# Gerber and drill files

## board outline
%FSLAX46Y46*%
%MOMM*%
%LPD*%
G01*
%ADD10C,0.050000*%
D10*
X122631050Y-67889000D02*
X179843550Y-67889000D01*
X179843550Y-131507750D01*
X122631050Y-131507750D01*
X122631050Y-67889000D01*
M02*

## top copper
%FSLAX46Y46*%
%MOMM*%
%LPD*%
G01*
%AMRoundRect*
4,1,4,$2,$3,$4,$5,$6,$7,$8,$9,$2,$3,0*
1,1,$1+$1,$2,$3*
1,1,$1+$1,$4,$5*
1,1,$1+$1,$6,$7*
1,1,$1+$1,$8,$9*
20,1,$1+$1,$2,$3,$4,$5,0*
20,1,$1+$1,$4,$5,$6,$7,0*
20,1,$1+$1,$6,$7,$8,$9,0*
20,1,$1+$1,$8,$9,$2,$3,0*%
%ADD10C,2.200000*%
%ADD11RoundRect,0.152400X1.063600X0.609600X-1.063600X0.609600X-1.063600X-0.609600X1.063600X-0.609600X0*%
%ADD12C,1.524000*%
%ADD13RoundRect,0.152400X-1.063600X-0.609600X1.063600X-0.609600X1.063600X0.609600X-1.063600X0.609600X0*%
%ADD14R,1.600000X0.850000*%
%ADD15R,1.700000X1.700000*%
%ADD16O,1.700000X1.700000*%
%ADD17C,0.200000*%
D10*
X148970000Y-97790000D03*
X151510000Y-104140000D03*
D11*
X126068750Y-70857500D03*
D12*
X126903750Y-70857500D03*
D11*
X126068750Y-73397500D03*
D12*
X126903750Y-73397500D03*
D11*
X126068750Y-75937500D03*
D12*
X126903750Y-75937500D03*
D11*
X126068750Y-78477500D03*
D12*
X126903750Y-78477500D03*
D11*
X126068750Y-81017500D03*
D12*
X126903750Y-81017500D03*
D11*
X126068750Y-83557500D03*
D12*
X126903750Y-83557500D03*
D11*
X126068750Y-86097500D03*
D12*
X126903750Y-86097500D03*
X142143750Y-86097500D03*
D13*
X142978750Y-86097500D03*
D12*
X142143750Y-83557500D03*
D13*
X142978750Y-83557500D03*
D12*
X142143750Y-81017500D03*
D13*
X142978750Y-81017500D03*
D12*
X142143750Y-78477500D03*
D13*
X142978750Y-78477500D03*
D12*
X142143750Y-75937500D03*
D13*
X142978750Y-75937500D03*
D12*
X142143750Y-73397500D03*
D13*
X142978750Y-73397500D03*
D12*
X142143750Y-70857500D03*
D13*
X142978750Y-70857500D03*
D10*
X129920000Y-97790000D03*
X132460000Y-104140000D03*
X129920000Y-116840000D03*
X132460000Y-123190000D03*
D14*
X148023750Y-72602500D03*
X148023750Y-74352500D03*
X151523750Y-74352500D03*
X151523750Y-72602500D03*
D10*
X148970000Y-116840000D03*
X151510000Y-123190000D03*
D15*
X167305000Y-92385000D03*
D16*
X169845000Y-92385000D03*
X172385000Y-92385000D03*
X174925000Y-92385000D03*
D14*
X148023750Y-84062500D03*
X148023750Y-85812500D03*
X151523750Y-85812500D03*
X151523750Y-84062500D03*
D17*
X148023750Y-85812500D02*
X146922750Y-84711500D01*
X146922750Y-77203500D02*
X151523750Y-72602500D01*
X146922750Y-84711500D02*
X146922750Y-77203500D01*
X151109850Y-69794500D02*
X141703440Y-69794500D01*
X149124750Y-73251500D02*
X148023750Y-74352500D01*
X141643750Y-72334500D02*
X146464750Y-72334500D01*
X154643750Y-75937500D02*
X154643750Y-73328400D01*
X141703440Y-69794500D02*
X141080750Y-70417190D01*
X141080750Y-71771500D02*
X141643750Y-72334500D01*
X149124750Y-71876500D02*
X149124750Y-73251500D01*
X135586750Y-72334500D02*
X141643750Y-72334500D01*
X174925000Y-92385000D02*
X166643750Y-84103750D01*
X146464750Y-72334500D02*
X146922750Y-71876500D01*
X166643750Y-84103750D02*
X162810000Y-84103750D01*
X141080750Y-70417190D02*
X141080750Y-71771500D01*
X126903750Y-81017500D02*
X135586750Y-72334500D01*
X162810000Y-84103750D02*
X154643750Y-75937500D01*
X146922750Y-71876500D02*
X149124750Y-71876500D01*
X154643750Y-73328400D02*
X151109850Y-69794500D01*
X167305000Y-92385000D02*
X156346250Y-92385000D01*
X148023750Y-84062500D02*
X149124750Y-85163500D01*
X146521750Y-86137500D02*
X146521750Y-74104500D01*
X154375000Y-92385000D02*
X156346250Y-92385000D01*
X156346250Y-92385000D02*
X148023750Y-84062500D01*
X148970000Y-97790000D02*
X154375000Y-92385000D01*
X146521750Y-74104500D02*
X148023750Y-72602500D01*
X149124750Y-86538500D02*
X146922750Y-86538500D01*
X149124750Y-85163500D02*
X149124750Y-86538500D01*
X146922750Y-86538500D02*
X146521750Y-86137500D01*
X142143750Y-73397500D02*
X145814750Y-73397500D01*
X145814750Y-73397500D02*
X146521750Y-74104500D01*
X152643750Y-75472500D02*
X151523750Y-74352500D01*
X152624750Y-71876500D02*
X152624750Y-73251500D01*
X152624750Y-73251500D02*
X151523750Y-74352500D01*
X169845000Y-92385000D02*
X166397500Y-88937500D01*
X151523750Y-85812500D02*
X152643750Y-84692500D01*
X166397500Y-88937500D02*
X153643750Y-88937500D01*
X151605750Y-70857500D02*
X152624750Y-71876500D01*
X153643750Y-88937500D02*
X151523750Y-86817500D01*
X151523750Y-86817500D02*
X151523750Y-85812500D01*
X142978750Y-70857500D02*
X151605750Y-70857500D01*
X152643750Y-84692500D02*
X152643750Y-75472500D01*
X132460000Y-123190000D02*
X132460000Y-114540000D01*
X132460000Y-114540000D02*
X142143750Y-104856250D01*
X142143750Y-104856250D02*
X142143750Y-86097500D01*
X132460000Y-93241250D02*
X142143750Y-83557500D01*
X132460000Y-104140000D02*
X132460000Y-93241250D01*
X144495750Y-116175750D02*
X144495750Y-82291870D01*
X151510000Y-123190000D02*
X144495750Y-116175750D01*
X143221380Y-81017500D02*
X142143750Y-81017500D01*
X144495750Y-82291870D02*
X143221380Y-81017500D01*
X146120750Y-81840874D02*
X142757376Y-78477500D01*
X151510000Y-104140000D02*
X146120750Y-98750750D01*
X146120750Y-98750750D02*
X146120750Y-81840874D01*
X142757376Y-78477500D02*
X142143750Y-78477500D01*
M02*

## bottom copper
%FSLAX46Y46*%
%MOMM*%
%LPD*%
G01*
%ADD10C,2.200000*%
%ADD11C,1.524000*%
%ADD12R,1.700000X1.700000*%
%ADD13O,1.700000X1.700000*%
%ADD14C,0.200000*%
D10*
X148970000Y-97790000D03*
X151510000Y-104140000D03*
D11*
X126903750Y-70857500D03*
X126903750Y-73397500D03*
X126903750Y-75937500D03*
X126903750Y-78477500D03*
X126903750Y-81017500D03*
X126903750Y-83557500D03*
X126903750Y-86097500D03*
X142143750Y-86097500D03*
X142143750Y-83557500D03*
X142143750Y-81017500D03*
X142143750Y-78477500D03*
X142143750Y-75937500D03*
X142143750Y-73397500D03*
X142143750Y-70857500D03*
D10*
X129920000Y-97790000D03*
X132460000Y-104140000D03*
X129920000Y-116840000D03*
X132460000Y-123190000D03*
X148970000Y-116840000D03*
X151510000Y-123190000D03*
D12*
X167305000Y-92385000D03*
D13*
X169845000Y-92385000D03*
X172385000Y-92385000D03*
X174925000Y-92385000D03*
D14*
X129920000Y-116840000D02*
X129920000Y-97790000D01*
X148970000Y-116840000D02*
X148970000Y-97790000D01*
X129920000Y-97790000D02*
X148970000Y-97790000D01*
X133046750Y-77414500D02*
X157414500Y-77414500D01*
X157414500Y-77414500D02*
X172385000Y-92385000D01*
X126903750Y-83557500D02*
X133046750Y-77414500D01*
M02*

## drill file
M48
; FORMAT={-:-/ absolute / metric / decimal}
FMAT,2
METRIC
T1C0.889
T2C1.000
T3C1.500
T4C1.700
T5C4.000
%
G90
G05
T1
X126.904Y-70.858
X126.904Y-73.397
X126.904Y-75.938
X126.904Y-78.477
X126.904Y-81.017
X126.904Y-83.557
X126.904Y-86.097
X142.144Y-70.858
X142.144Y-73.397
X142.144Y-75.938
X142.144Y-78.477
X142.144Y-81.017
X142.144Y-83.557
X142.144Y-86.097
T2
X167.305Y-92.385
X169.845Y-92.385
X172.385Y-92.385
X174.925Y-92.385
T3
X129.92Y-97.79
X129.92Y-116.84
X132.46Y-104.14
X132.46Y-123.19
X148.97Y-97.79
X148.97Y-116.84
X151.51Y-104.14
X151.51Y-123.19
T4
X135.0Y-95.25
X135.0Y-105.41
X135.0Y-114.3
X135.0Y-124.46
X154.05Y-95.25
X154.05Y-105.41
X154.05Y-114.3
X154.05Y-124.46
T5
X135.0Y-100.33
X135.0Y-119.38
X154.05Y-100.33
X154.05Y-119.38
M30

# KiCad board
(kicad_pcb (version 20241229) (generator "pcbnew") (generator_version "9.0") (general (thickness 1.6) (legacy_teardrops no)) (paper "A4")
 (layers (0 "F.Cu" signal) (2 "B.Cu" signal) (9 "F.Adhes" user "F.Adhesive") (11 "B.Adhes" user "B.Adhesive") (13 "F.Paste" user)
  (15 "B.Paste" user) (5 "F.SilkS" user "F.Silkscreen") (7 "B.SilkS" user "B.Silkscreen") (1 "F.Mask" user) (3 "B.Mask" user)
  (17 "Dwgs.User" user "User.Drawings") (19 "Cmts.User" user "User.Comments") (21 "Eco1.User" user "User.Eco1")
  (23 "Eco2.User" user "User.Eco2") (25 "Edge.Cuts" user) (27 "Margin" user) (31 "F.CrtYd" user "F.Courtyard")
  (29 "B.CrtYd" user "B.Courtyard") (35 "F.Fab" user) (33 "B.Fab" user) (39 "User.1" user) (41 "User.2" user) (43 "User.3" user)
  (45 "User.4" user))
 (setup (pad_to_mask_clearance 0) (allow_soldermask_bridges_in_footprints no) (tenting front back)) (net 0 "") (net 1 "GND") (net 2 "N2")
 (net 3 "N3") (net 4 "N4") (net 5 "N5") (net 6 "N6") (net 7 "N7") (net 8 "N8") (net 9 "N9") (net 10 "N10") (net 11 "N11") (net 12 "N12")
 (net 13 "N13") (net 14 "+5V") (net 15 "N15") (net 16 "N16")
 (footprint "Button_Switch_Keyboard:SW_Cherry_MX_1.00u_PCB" (layer "F.Cu") (at 148.97 97.79 90)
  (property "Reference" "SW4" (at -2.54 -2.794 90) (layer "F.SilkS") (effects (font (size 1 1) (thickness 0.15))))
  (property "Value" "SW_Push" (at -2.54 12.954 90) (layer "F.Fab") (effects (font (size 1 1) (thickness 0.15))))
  (pad "" np_thru_hole circle (at -7.62 5.08 90) (size 1.7 1.7) (drill 1.7) (layers "*.Cu" "*.Mask"))
  (pad "" np_thru_hole circle (at -2.54 5.08 90) (size 4 4) (drill 4) (layers "*.Cu" "*.Mask"))
  (pad "" np_thru_hole circle (at 2.54 5.08 90) (size 1.7 1.7) (drill 1.7) (layers "*.Cu" "*.Mask"))
  (pad "1" thru_hole circle (at 0 0 90) (size 2.2 2.2) (drill 1.5) (layers "*.Cu" "*.Mask") (remove_unused_layers no) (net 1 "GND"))
  (pad "2" thru_hole circle (at -6.35 2.54 90) (size 2.2 2.2) (drill 1.5) (layers "*.Cu" "*.Mask") (remove_unused_layers no) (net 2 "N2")))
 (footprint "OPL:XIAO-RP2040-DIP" (layer "F.Cu") (at 134.52375 78.4775)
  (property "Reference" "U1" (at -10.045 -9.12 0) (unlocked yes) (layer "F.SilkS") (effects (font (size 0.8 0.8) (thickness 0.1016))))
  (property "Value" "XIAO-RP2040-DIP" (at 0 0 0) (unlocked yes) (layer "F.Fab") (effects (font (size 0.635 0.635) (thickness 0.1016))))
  (pad "1" smd roundrect (at -8.455 -7.62 180) (size 2.432 1.524) (layers "F.Cu" "F.Mask") (roundrect_rratio 0.1) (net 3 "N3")
   (thermal_bridge_angle 45))
  (pad "1" thru_hole circle (at -7.62 -7.62 180) (size 1.524 1.524) (drill 0.889) (layers "*.Cu" "*.Mask") (remove_unused_layers no)
   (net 3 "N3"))
  (pad "2" smd roundrect (at -8.455 -5.08 180) (size 2.432 1.524) (layers "F.Cu" "F.Mask") (roundrect_rratio 0.1) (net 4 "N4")
   (thermal_bridge_angle 45))
  (pad "2" thru_hole circle (at -7.62 -5.08 180) (size 1.524 1.524) (drill 0.889) (layers "*.Cu" "*.Mask") (remove_unused_layers no)
   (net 4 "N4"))
  (pad "3" smd roundrect (at -8.455 -2.54 180) (size 2.432 1.524) (layers "F.Cu" "F.Mask") (roundrect_rratio 0.1) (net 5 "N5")
   (thermal_bridge_angle 45))
  (pad "3" thru_hole circle (at -7.62 -2.54 180) (size 1.524 1.524) (drill 0.889) (layers "*.Cu" "*.Mask") (remove_unused_layers no)
   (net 5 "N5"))
  (pad "4" smd roundrect (at -8.455 0 180) (size 2.432 1.524) (layers "F.Cu" "F.Mask") (roundrect_rratio 0.1) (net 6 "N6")
   (thermal_bridge_angle 45))
  (pad "4" thru_hole circle (at -7.62 0 180) (size 1.524 1.524) (drill 0.889) (layers "*.Cu" "*.Mask") (remove_unused_layers no)
   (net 6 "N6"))
  (pad "5" smd roundrect (at -8.455 2.54 180) (size 2.432 1.524) (layers "F.Cu" "F.Mask") (roundrect_rratio 0.1) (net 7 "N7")
   (thermal_bridge_angle 45))
  (pad "5" thru_hole circle (at -7.62 2.54 180) (size 1.524 1.524) (drill 0.889) (layers "*.Cu" "*.Mask") (remove_unused_layers no)
   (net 7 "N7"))
  (pad "6" smd roundrect (at -8.455 5.08 180) (size 2.432 1.524) (layers "F.Cu" "F.Mask") (roundrect_rratio 0.1) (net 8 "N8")
   (thermal_bridge_angle 45))
  (pad "6" thru_hole circle (at -7.62 5.08 180) (size 1.524 1.524) (drill 0.889) (layers "*.Cu" "*.Mask") (remove_unused_layers no)
   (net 8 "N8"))
  (pad "7" smd roundrect (at -8.455 7.62 180) (size 2.432 1.524) (layers "F.Cu" "F.Mask") (roundrect_rratio 0.1) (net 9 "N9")
   (thermal_bridge_angle 45))
  (pad "7" thru_hole circle (at -7.62 7.62 180) (size 1.524 1.524) (drill 0.889) (layers "*.Cu" "*.Mask") (remove_unused_layers no)
   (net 9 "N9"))
  (pad "8" thru_hole circle (at 7.62 7.62) (size 1.524 1.524) (drill 0.889) (layers "*.Cu" "*.Mask") (remove_unused_layers no)
   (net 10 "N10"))
  (pad "8" smd roundrect (at 8.455 7.62) (size 2.432 1.524) (layers "F.Cu" "F.Mask") (roundrect_rratio 0.1) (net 10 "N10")
   (thermal_bridge_angle 45))
  (pad "9" thru_hole circle (at 7.62 5.08) (size 1.524 1.524) (drill 0.889) (layers "*.Cu" "*.Mask") (remove_unused_layers no)
   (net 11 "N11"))
  (pad "9" smd roundrect (at 8.455 5.08) (size 2.432 1.524) (layers "F.Cu" "F.Mask") (roundrect_rratio 0.1) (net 11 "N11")
   (thermal_bridge_angle 45))
  (pad "10" thru_hole circle (at 7.62 2.54) (size 1.524 1.524) (drill 0.889) (layers "*.Cu" "*.Mask") (remove_unused_layers no)
   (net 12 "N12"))
  (pad "10" smd roundrect (at 8.455 2.54) (size 2.432 1.524) (layers "F.Cu" "F.Mask") (roundrect_rratio 0.1) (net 12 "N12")
   (thermal_bridge_angle 45))
  (pad "11" thru_hole circle (at 7.62 0) (size 1.524 1.524) (drill 0.889) (layers "*.Cu" "*.Mask") (remove_unused_layers no) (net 2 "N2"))
  (pad "11" smd roundrect (at 8.455 0) (size 2.432 1.524) (layers "F.Cu" "F.Mask") (roundrect_rratio 0.1) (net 2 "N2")
   (thermal_bridge_angle 45))
  (pad "12" thru_hole circle (at 7.62 -2.54) (size 1.524 1.524) (drill 0.889) (layers "*.Cu" "*.Mask") (remove_unused_layers no)
   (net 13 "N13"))
  (pad "12" smd roundrect (at 8.455 -2.54) (size 2.432 1.524) (layers "F.Cu" "F.Mask") (roundrect_rratio 0.1) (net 13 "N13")
   (thermal_bridge_angle 45))
  (pad "13" thru_hole circle (at 7.62 -5.08) (size 1.524 1.524) (drill 0.889) (layers "*.Cu" "*.Mask") (remove_unused_layers no)
   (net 1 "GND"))
  (pad "13" smd roundrect (at 8.455 -5.08) (size 2.432 1.524) (layers "F.Cu" "F.Mask") (roundrect_rratio 0.1) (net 1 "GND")
   (thermal_bridge_angle 45))
  (pad "14" thru_hole circle (at 7.62 -7.62) (size 1.524 1.524) (drill 0.889) (layers "*.Cu" "*.Mask") (remove_unused_layers no)
   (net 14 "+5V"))
  (pad "14" smd roundrect (at 8.455 -7.62) (size 2.432 1.524) (layers "F.Cu" "F.Mask") (roundrect_rratio 0.1) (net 14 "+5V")
   (thermal_bridge_angle 45)))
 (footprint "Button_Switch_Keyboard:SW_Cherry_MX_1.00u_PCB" (layer "F.Cu") (at 129.92 97.79 90)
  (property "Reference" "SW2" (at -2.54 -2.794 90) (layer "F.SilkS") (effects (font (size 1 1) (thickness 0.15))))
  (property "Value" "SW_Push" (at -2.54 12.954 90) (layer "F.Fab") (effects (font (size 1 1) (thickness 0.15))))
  (pad "" np_thru_hole circle (at -7.62 5.08 90) (size 1.7 1.7) (drill 1.7) (layers "*.Cu" "*.Mask"))
  (pad "" np_thru_hole circle (at -2.54 5.08 90) (size 4 4) (drill 4) (layers "*.Cu" "*.Mask"))
  (pad "" np_thru_hole circle (at 2.54 5.08 90) (size 1.7 1.7) (drill 1.7) (layers "*.Cu" "*.Mask"))
  (pad "1" thru_hole circle (at 0 0 90) (size 2.2 2.2) (drill 1.5) (layers "*.Cu" "*.Mask") (remove_unused_layers no) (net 1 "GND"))
  (pad "2" thru_hole circle (at -6.35 2.54 90) (size 2.2 2.2) (drill 1.5) (layers "*.Cu" "*.Mask") (remove_unused_layers no) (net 11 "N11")))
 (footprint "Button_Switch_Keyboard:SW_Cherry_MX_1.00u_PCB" (layer "F.Cu") (at 129.92 116.84 90)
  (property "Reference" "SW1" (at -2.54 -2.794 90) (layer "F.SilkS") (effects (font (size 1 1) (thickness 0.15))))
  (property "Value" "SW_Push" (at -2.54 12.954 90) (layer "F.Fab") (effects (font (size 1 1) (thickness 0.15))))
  (pad "" np_thru_hole circle (at -7.62 5.08 90) (size 1.7 1.7) (drill 1.7) (layers "*.Cu" "*.Mask"))
  (pad "" np_thru_hole circle (at -2.54 5.08 90) (size 4 4) (drill 4) (layers "*.Cu" "*.Mask"))
  (pad "" np_thru_hole circle (at 2.54 5.08 90) (size 1.7 1.7) (drill 1.7) (layers "*.Cu" "*.Mask"))
  (pad "1" thru_hole circle (at 0 0 90) (size 2.2 2.2) (drill 1.5) (layers "*.Cu" "*.Mask") (remove_unused_layers no) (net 1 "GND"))
  (pad "2" thru_hole circle (at -6.35 2.54 90) (size 2.2 2.2) (drill 1.5) (layers "*.Cu" "*.Mask") (remove_unused_layers no) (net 10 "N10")))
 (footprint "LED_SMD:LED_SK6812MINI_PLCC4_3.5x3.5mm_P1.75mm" (layer "F.Cu") (at 149.77375 73.4775)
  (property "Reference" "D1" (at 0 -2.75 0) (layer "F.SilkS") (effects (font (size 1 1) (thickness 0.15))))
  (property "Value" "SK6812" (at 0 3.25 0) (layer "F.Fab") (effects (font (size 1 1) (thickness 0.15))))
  (pad "1" smd rect (at -1.75 -0.875) (size 1.6 0.85) (layers "F.Cu" "F.Mask" "F.Paste") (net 1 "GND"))
  (pad "2" smd rect (at -1.75 0.875) (size 1.6 0.85) (layers "F.Cu" "F.Mask" "F.Paste") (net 7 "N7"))
  (pad "3" smd rect (at 1.75 0.875) (size 1.6 0.85) (layers "F.Cu" "F.Mask" "F.Paste") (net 14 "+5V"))
  (pad "4" smd rect (at 1.75 -0.875) (size 1.6 0.85) (layers "F.Cu" "F.Mask" "F.Paste") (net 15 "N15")))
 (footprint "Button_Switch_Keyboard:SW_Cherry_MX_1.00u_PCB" (layer "F.Cu") (at 148.97 116.84 90)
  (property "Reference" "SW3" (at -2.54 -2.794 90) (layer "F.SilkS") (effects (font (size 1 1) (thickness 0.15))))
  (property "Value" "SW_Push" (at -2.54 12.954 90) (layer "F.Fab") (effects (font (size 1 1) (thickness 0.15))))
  (pad "" np_thru_hole circle (at -7.62 5.08 90) (size 1.7 1.7) (drill 1.7) (layers "*.Cu" "*.Mask"))
  (pad "" np_thru_hole circle (at -2.54 5.08 90) (size 4 4) (drill 4) (layers "*.Cu" "*.Mask"))
  (pad "" np_thru_hole circle (at 2.54 5.08 90) (size 1.7 1.7) (drill 1.7) (layers "*.Cu" "*.Mask"))
  (pad "1" thru_hole circle (at 0 0 90) (size 2.2 2.2) (drill 1.5) (layers "*.Cu" "*.Mask") (remove_unused_layers no) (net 1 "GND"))
  (pad "2" thru_hole circle (at -6.35 2.54 90) (size 2.2 2.2) (drill 1.5) (layers "*.Cu" "*.Mask") (remove_unused_layers no) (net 12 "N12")))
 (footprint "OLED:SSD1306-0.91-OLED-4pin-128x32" (layer "F.Cu") (at 165.115 128.885 90)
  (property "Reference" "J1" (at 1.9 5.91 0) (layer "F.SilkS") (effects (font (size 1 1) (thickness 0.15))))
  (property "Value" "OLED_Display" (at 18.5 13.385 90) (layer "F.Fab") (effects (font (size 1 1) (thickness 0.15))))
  (pad "1" thru_hole rect (at 36.5 2.19 90) (size 1.7 1.7) (drill 1) (layers "*.Cu" "*.Mask") (remove_unused_layers no) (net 1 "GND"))
  (pad "2" thru_hole oval (at 36.5 4.73 90) (size 1.7 1.7) (drill 1) (layers "*.Cu" "*.Mask") (remove_unused_layers no) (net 14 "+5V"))
  (pad "3" thru_hole oval (at 36.5 7.27 90) (size 1.7 1.7) (drill 1) (layers "*.Cu" "*.Mask") (remove_unused_layers no) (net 8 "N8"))
  (pad "4" thru_hole oval (at 36.5 9.81 90) (size 1.7 1.7) (drill 1) (layers "*.Cu" "*.Mask") (remove_unused_layers no) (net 7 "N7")))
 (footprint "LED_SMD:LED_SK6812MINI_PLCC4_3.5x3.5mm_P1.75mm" (layer "F.Cu") (at 149.77375 84.9375)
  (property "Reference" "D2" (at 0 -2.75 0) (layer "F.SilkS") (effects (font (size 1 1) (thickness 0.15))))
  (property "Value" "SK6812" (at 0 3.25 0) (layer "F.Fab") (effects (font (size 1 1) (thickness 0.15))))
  (pad "1" smd rect (at -1.75 -0.875) (size 1.6 0.85) (layers "F.Cu" "F.Mask" "F.Paste") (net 1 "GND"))
  (pad "2" smd rect (at -1.75 0.875) (size 1.6 0.85) (layers "F.Cu" "F.Mask" "F.Paste") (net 15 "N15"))
  (pad "3" smd rect (at 1.75 0.875) (size 1.6 0.85) (layers "F.Cu" "F.Mask" "F.Paste") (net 14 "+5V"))
  (pad "4" smd rect (at 1.75 -0.875) (size 1.6 0.85) (layers "F.Cu" "F.Mask" "F.Paste") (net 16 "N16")))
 (gr_rect (start 122.63105 67.889) (end 179.84355 131.50775) (stroke (width 0.05) (type solid)) (fill no) (layer "Edge.Cuts"))
 (segment (start 148.02375 85.8125) (end 146.92275 84.7115) (width 0.2) (layer "F.Cu") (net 15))
 (segment (start 146.92275 77.2035) (end 151.52375 72.6025) (width 0.2) (layer "F.Cu") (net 15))
 (segment (start 146.92275 84.7115) (end 146.92275 77.2035) (width 0.2) (layer "F.Cu") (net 15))
 (segment (start 151.10985 69.7945) (end 141.70344 69.7945) (width 0.2) (layer "F.Cu") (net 7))
 (segment (start 149.12475 73.2515) (end 148.02375 74.3525) (width 0.2) (layer "F.Cu") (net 7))
 (segment (start 141.64375 72.3345) (end 146.46475 72.3345) (width 0.2) (layer "F.Cu") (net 7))
 (segment (start 154.64375 75.9375) (end 154.64375 73.3284) (width 0.2) (layer "F.Cu") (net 7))
 (segment (start 141.70344 69.7945) (end 141.08075 70.41719) (width 0.2) (layer "F.Cu") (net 7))
 (segment (start 141.08075 71.7715) (end 141.64375 72.3345) (width 0.2) (layer "F.Cu") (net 7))
 (segment (start 149.12475 71.8765) (end 149.12475 73.2515) (width 0.2) (layer "F.Cu") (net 7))
 (segment (start 135.58675 72.3345) (end 141.64375 72.3345) (width 0.2) (layer "F.Cu") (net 7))
 (segment (start 174.925 92.385) (end 166.64375 84.10375) (width 0.2) (layer "F.Cu") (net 7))
 (segment (start 146.46475 72.3345) (end 146.92275 71.8765) (width 0.2) (layer "F.Cu") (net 7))
 (segment (start 166.64375 84.10375) (end 162.81 84.10375) (width 0.2) (layer "F.Cu") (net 7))
 (segment (start 141.08075 70.41719) (end 141.08075 71.7715) (width 0.2) (layer "F.Cu") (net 7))
 (segment (start 126.90375 81.0175) (end 135.58675 72.3345) (width 0.2) (layer "F.Cu") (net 7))
 (segment (start 162.81 84.10375) (end 154.64375 75.9375) (width 0.2) (layer "F.Cu") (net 7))
 (segment (start 146.92275 71.8765) (end 149.12475 71.8765) (width 0.2) (layer "F.Cu") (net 7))
 (segment (start 154.64375 73.3284) (end 151.10985 69.7945) (width 0.2) (layer "F.Cu") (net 7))
 (segment (start 167.305 92.385) (end 156.34625 92.385) (width 0.2) (layer "F.Cu") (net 1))
 (segment (start 148.02375 84.0625) (end 149.12475 85.1635) (width 0.2) (layer "F.Cu") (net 1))
 (segment (start 146.52175 86.1375) (end 146.52175 74.1045) (width 0.2) (layer "F.Cu") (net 1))
 (segment (start 154.375 92.385) (end 156.34625 92.385) (width 0.2) (layer "F.Cu") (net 1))
 (segment (start 156.34625 92.385) (end 148.02375 84.0625) (width 0.2) (layer "F.Cu") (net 1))
 (segment (start 148.97 97.79) (end 154.375 92.385) (width 0.2) (layer "F.Cu") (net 1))
 (segment (start 146.52175 74.1045) (end 148.02375 72.6025) (width 0.2) (layer "F.Cu") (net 1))
 (segment (start 149.12475 86.5385) (end 146.92275 86.5385) (width 0.2) (layer "F.Cu") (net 1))
 (segment (start 149.12475 85.1635) (end 149.12475 86.5385) (width 0.2) (layer "F.Cu") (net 1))
 (segment (start 146.92275 86.5385) (end 146.52175 86.1375) (width 0.2) (layer "F.Cu") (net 1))
 (segment (start 142.14375 73.3975) (end 145.81475 73.3975) (width 0.2) (layer "F.Cu") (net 1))
 (segment (start 145.81475 73.3975) (end 146.52175 74.1045) (width 0.2) (layer "F.Cu") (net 1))
 (segment (start 129.92 116.84) (end 129.92 97.79) (width 0.2) (layer "B.Cu") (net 1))
 (segment (start 148.97 116.84) (end 148.97 97.79) (width 0.2) (layer "B.Cu") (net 1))
 (segment (start 129.92 97.79) (end 148.97 97.79) (width 0.2) (layer "B.Cu") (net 1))
 (segment (start 152.64375 75.4725) (end 151.52375 74.3525) (width 0.2) (layer "F.Cu") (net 14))
 (segment (start 152.62475 71.8765) (end 152.62475 73.2515) (width 0.2) (layer "F.Cu") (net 14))
 (segment (start 152.62475 73.2515) (end 151.52375 74.3525) (width 0.2) (layer "F.Cu") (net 14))
 (segment (start 169.845 92.385) (end 166.3975 88.9375) (width 0.2) (layer "F.Cu") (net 14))
 (segment (start 151.52375 85.8125) (end 152.64375 84.6925) (width 0.2) (layer "F.Cu") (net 14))
 (segment (start 166.3975 88.9375) (end 153.64375 88.9375) (width 0.2) (layer "F.Cu") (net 14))
 (segment (start 151.60575 70.8575) (end 152.62475 71.8765) (width 0.2) (layer "F.Cu") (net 14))
 (segment (start 153.64375 88.9375) (end 151.52375 86.8175) (width 0.2) (layer "F.Cu") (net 14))
 (segment (start 151.52375 86.8175) (end 151.52375 85.8125) (width 0.2) (layer "F.Cu") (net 14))
 (segment (start 142.97875 70.8575) (end 151.60575 70.8575) (width 0.2) (layer "F.Cu") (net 14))
 (segment (start 152.64375 84.6925) (end 152.64375 75.4725) (width 0.2) (layer "F.Cu") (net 14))
 (segment (start 132.46 123.19) (end 132.46 114.54) (width 0.2) (layer "F.Cu") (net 10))
 (segment (start 132.46 114.54) (end 142.14375 104.85625) (width 0.2) (layer "F.Cu") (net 10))
 (segment (start 142.14375 104.85625) (end 142.14375 86.0975) (width 0.2) (layer "F.Cu") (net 10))
 (segment (start 132.46 93.24125) (end 142.14375 83.5575) (width 0.2) (layer "F.Cu") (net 11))
 (segment (start 132.46 104.14) (end 132.46 93.24125) (width 0.2) (layer "F.Cu") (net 11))
 (segment (start 144.49575 116.17575) (end 144.49575 82.29187) (width 0.2) (layer "F.Cu") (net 12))
 (segment (start 151.51 123.19) (end 144.49575 116.17575) (width 0.2) (layer "F.Cu") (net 12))
 (segment (start 143.22138 81.0175) (end 142.14375 81.0175) (width 0.2) (layer "F.Cu") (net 12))
 (segment (start 144.49575 82.29187) (end 143.22138 81.0175) (width 0.2) (layer "F.Cu") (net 12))
 (segment (start 146.12075 81.840874) (end 142.757376 78.4775) (width 0.2) (layer "F.Cu") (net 2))
 (segment (start 151.51 104.14) (end 146.12075 98.75075) (width 0.2) (layer "F.Cu") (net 2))
 (segment (start 146.12075 98.75075) (end 146.12075 81.840874) (width 0.2) (layer "F.Cu") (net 2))
 (segment (start 142.757376 78.4775) (end 142.14375 78.4775) (width 0.2) (layer "F.Cu") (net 2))
 (segment (start 133.04675 77.4145) (end 157.4145 77.4145) (width 0.2) (layer "B.Cu") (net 8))
 (segment (start 157.4145 77.4145) (end 172.385 92.385) (width 0.2) (layer "B.Cu") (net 8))
 (segment (start 126.90375 83.5575) (end 133.04675 77.4145) (width 0.2) (layer "B.Cu") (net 8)))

